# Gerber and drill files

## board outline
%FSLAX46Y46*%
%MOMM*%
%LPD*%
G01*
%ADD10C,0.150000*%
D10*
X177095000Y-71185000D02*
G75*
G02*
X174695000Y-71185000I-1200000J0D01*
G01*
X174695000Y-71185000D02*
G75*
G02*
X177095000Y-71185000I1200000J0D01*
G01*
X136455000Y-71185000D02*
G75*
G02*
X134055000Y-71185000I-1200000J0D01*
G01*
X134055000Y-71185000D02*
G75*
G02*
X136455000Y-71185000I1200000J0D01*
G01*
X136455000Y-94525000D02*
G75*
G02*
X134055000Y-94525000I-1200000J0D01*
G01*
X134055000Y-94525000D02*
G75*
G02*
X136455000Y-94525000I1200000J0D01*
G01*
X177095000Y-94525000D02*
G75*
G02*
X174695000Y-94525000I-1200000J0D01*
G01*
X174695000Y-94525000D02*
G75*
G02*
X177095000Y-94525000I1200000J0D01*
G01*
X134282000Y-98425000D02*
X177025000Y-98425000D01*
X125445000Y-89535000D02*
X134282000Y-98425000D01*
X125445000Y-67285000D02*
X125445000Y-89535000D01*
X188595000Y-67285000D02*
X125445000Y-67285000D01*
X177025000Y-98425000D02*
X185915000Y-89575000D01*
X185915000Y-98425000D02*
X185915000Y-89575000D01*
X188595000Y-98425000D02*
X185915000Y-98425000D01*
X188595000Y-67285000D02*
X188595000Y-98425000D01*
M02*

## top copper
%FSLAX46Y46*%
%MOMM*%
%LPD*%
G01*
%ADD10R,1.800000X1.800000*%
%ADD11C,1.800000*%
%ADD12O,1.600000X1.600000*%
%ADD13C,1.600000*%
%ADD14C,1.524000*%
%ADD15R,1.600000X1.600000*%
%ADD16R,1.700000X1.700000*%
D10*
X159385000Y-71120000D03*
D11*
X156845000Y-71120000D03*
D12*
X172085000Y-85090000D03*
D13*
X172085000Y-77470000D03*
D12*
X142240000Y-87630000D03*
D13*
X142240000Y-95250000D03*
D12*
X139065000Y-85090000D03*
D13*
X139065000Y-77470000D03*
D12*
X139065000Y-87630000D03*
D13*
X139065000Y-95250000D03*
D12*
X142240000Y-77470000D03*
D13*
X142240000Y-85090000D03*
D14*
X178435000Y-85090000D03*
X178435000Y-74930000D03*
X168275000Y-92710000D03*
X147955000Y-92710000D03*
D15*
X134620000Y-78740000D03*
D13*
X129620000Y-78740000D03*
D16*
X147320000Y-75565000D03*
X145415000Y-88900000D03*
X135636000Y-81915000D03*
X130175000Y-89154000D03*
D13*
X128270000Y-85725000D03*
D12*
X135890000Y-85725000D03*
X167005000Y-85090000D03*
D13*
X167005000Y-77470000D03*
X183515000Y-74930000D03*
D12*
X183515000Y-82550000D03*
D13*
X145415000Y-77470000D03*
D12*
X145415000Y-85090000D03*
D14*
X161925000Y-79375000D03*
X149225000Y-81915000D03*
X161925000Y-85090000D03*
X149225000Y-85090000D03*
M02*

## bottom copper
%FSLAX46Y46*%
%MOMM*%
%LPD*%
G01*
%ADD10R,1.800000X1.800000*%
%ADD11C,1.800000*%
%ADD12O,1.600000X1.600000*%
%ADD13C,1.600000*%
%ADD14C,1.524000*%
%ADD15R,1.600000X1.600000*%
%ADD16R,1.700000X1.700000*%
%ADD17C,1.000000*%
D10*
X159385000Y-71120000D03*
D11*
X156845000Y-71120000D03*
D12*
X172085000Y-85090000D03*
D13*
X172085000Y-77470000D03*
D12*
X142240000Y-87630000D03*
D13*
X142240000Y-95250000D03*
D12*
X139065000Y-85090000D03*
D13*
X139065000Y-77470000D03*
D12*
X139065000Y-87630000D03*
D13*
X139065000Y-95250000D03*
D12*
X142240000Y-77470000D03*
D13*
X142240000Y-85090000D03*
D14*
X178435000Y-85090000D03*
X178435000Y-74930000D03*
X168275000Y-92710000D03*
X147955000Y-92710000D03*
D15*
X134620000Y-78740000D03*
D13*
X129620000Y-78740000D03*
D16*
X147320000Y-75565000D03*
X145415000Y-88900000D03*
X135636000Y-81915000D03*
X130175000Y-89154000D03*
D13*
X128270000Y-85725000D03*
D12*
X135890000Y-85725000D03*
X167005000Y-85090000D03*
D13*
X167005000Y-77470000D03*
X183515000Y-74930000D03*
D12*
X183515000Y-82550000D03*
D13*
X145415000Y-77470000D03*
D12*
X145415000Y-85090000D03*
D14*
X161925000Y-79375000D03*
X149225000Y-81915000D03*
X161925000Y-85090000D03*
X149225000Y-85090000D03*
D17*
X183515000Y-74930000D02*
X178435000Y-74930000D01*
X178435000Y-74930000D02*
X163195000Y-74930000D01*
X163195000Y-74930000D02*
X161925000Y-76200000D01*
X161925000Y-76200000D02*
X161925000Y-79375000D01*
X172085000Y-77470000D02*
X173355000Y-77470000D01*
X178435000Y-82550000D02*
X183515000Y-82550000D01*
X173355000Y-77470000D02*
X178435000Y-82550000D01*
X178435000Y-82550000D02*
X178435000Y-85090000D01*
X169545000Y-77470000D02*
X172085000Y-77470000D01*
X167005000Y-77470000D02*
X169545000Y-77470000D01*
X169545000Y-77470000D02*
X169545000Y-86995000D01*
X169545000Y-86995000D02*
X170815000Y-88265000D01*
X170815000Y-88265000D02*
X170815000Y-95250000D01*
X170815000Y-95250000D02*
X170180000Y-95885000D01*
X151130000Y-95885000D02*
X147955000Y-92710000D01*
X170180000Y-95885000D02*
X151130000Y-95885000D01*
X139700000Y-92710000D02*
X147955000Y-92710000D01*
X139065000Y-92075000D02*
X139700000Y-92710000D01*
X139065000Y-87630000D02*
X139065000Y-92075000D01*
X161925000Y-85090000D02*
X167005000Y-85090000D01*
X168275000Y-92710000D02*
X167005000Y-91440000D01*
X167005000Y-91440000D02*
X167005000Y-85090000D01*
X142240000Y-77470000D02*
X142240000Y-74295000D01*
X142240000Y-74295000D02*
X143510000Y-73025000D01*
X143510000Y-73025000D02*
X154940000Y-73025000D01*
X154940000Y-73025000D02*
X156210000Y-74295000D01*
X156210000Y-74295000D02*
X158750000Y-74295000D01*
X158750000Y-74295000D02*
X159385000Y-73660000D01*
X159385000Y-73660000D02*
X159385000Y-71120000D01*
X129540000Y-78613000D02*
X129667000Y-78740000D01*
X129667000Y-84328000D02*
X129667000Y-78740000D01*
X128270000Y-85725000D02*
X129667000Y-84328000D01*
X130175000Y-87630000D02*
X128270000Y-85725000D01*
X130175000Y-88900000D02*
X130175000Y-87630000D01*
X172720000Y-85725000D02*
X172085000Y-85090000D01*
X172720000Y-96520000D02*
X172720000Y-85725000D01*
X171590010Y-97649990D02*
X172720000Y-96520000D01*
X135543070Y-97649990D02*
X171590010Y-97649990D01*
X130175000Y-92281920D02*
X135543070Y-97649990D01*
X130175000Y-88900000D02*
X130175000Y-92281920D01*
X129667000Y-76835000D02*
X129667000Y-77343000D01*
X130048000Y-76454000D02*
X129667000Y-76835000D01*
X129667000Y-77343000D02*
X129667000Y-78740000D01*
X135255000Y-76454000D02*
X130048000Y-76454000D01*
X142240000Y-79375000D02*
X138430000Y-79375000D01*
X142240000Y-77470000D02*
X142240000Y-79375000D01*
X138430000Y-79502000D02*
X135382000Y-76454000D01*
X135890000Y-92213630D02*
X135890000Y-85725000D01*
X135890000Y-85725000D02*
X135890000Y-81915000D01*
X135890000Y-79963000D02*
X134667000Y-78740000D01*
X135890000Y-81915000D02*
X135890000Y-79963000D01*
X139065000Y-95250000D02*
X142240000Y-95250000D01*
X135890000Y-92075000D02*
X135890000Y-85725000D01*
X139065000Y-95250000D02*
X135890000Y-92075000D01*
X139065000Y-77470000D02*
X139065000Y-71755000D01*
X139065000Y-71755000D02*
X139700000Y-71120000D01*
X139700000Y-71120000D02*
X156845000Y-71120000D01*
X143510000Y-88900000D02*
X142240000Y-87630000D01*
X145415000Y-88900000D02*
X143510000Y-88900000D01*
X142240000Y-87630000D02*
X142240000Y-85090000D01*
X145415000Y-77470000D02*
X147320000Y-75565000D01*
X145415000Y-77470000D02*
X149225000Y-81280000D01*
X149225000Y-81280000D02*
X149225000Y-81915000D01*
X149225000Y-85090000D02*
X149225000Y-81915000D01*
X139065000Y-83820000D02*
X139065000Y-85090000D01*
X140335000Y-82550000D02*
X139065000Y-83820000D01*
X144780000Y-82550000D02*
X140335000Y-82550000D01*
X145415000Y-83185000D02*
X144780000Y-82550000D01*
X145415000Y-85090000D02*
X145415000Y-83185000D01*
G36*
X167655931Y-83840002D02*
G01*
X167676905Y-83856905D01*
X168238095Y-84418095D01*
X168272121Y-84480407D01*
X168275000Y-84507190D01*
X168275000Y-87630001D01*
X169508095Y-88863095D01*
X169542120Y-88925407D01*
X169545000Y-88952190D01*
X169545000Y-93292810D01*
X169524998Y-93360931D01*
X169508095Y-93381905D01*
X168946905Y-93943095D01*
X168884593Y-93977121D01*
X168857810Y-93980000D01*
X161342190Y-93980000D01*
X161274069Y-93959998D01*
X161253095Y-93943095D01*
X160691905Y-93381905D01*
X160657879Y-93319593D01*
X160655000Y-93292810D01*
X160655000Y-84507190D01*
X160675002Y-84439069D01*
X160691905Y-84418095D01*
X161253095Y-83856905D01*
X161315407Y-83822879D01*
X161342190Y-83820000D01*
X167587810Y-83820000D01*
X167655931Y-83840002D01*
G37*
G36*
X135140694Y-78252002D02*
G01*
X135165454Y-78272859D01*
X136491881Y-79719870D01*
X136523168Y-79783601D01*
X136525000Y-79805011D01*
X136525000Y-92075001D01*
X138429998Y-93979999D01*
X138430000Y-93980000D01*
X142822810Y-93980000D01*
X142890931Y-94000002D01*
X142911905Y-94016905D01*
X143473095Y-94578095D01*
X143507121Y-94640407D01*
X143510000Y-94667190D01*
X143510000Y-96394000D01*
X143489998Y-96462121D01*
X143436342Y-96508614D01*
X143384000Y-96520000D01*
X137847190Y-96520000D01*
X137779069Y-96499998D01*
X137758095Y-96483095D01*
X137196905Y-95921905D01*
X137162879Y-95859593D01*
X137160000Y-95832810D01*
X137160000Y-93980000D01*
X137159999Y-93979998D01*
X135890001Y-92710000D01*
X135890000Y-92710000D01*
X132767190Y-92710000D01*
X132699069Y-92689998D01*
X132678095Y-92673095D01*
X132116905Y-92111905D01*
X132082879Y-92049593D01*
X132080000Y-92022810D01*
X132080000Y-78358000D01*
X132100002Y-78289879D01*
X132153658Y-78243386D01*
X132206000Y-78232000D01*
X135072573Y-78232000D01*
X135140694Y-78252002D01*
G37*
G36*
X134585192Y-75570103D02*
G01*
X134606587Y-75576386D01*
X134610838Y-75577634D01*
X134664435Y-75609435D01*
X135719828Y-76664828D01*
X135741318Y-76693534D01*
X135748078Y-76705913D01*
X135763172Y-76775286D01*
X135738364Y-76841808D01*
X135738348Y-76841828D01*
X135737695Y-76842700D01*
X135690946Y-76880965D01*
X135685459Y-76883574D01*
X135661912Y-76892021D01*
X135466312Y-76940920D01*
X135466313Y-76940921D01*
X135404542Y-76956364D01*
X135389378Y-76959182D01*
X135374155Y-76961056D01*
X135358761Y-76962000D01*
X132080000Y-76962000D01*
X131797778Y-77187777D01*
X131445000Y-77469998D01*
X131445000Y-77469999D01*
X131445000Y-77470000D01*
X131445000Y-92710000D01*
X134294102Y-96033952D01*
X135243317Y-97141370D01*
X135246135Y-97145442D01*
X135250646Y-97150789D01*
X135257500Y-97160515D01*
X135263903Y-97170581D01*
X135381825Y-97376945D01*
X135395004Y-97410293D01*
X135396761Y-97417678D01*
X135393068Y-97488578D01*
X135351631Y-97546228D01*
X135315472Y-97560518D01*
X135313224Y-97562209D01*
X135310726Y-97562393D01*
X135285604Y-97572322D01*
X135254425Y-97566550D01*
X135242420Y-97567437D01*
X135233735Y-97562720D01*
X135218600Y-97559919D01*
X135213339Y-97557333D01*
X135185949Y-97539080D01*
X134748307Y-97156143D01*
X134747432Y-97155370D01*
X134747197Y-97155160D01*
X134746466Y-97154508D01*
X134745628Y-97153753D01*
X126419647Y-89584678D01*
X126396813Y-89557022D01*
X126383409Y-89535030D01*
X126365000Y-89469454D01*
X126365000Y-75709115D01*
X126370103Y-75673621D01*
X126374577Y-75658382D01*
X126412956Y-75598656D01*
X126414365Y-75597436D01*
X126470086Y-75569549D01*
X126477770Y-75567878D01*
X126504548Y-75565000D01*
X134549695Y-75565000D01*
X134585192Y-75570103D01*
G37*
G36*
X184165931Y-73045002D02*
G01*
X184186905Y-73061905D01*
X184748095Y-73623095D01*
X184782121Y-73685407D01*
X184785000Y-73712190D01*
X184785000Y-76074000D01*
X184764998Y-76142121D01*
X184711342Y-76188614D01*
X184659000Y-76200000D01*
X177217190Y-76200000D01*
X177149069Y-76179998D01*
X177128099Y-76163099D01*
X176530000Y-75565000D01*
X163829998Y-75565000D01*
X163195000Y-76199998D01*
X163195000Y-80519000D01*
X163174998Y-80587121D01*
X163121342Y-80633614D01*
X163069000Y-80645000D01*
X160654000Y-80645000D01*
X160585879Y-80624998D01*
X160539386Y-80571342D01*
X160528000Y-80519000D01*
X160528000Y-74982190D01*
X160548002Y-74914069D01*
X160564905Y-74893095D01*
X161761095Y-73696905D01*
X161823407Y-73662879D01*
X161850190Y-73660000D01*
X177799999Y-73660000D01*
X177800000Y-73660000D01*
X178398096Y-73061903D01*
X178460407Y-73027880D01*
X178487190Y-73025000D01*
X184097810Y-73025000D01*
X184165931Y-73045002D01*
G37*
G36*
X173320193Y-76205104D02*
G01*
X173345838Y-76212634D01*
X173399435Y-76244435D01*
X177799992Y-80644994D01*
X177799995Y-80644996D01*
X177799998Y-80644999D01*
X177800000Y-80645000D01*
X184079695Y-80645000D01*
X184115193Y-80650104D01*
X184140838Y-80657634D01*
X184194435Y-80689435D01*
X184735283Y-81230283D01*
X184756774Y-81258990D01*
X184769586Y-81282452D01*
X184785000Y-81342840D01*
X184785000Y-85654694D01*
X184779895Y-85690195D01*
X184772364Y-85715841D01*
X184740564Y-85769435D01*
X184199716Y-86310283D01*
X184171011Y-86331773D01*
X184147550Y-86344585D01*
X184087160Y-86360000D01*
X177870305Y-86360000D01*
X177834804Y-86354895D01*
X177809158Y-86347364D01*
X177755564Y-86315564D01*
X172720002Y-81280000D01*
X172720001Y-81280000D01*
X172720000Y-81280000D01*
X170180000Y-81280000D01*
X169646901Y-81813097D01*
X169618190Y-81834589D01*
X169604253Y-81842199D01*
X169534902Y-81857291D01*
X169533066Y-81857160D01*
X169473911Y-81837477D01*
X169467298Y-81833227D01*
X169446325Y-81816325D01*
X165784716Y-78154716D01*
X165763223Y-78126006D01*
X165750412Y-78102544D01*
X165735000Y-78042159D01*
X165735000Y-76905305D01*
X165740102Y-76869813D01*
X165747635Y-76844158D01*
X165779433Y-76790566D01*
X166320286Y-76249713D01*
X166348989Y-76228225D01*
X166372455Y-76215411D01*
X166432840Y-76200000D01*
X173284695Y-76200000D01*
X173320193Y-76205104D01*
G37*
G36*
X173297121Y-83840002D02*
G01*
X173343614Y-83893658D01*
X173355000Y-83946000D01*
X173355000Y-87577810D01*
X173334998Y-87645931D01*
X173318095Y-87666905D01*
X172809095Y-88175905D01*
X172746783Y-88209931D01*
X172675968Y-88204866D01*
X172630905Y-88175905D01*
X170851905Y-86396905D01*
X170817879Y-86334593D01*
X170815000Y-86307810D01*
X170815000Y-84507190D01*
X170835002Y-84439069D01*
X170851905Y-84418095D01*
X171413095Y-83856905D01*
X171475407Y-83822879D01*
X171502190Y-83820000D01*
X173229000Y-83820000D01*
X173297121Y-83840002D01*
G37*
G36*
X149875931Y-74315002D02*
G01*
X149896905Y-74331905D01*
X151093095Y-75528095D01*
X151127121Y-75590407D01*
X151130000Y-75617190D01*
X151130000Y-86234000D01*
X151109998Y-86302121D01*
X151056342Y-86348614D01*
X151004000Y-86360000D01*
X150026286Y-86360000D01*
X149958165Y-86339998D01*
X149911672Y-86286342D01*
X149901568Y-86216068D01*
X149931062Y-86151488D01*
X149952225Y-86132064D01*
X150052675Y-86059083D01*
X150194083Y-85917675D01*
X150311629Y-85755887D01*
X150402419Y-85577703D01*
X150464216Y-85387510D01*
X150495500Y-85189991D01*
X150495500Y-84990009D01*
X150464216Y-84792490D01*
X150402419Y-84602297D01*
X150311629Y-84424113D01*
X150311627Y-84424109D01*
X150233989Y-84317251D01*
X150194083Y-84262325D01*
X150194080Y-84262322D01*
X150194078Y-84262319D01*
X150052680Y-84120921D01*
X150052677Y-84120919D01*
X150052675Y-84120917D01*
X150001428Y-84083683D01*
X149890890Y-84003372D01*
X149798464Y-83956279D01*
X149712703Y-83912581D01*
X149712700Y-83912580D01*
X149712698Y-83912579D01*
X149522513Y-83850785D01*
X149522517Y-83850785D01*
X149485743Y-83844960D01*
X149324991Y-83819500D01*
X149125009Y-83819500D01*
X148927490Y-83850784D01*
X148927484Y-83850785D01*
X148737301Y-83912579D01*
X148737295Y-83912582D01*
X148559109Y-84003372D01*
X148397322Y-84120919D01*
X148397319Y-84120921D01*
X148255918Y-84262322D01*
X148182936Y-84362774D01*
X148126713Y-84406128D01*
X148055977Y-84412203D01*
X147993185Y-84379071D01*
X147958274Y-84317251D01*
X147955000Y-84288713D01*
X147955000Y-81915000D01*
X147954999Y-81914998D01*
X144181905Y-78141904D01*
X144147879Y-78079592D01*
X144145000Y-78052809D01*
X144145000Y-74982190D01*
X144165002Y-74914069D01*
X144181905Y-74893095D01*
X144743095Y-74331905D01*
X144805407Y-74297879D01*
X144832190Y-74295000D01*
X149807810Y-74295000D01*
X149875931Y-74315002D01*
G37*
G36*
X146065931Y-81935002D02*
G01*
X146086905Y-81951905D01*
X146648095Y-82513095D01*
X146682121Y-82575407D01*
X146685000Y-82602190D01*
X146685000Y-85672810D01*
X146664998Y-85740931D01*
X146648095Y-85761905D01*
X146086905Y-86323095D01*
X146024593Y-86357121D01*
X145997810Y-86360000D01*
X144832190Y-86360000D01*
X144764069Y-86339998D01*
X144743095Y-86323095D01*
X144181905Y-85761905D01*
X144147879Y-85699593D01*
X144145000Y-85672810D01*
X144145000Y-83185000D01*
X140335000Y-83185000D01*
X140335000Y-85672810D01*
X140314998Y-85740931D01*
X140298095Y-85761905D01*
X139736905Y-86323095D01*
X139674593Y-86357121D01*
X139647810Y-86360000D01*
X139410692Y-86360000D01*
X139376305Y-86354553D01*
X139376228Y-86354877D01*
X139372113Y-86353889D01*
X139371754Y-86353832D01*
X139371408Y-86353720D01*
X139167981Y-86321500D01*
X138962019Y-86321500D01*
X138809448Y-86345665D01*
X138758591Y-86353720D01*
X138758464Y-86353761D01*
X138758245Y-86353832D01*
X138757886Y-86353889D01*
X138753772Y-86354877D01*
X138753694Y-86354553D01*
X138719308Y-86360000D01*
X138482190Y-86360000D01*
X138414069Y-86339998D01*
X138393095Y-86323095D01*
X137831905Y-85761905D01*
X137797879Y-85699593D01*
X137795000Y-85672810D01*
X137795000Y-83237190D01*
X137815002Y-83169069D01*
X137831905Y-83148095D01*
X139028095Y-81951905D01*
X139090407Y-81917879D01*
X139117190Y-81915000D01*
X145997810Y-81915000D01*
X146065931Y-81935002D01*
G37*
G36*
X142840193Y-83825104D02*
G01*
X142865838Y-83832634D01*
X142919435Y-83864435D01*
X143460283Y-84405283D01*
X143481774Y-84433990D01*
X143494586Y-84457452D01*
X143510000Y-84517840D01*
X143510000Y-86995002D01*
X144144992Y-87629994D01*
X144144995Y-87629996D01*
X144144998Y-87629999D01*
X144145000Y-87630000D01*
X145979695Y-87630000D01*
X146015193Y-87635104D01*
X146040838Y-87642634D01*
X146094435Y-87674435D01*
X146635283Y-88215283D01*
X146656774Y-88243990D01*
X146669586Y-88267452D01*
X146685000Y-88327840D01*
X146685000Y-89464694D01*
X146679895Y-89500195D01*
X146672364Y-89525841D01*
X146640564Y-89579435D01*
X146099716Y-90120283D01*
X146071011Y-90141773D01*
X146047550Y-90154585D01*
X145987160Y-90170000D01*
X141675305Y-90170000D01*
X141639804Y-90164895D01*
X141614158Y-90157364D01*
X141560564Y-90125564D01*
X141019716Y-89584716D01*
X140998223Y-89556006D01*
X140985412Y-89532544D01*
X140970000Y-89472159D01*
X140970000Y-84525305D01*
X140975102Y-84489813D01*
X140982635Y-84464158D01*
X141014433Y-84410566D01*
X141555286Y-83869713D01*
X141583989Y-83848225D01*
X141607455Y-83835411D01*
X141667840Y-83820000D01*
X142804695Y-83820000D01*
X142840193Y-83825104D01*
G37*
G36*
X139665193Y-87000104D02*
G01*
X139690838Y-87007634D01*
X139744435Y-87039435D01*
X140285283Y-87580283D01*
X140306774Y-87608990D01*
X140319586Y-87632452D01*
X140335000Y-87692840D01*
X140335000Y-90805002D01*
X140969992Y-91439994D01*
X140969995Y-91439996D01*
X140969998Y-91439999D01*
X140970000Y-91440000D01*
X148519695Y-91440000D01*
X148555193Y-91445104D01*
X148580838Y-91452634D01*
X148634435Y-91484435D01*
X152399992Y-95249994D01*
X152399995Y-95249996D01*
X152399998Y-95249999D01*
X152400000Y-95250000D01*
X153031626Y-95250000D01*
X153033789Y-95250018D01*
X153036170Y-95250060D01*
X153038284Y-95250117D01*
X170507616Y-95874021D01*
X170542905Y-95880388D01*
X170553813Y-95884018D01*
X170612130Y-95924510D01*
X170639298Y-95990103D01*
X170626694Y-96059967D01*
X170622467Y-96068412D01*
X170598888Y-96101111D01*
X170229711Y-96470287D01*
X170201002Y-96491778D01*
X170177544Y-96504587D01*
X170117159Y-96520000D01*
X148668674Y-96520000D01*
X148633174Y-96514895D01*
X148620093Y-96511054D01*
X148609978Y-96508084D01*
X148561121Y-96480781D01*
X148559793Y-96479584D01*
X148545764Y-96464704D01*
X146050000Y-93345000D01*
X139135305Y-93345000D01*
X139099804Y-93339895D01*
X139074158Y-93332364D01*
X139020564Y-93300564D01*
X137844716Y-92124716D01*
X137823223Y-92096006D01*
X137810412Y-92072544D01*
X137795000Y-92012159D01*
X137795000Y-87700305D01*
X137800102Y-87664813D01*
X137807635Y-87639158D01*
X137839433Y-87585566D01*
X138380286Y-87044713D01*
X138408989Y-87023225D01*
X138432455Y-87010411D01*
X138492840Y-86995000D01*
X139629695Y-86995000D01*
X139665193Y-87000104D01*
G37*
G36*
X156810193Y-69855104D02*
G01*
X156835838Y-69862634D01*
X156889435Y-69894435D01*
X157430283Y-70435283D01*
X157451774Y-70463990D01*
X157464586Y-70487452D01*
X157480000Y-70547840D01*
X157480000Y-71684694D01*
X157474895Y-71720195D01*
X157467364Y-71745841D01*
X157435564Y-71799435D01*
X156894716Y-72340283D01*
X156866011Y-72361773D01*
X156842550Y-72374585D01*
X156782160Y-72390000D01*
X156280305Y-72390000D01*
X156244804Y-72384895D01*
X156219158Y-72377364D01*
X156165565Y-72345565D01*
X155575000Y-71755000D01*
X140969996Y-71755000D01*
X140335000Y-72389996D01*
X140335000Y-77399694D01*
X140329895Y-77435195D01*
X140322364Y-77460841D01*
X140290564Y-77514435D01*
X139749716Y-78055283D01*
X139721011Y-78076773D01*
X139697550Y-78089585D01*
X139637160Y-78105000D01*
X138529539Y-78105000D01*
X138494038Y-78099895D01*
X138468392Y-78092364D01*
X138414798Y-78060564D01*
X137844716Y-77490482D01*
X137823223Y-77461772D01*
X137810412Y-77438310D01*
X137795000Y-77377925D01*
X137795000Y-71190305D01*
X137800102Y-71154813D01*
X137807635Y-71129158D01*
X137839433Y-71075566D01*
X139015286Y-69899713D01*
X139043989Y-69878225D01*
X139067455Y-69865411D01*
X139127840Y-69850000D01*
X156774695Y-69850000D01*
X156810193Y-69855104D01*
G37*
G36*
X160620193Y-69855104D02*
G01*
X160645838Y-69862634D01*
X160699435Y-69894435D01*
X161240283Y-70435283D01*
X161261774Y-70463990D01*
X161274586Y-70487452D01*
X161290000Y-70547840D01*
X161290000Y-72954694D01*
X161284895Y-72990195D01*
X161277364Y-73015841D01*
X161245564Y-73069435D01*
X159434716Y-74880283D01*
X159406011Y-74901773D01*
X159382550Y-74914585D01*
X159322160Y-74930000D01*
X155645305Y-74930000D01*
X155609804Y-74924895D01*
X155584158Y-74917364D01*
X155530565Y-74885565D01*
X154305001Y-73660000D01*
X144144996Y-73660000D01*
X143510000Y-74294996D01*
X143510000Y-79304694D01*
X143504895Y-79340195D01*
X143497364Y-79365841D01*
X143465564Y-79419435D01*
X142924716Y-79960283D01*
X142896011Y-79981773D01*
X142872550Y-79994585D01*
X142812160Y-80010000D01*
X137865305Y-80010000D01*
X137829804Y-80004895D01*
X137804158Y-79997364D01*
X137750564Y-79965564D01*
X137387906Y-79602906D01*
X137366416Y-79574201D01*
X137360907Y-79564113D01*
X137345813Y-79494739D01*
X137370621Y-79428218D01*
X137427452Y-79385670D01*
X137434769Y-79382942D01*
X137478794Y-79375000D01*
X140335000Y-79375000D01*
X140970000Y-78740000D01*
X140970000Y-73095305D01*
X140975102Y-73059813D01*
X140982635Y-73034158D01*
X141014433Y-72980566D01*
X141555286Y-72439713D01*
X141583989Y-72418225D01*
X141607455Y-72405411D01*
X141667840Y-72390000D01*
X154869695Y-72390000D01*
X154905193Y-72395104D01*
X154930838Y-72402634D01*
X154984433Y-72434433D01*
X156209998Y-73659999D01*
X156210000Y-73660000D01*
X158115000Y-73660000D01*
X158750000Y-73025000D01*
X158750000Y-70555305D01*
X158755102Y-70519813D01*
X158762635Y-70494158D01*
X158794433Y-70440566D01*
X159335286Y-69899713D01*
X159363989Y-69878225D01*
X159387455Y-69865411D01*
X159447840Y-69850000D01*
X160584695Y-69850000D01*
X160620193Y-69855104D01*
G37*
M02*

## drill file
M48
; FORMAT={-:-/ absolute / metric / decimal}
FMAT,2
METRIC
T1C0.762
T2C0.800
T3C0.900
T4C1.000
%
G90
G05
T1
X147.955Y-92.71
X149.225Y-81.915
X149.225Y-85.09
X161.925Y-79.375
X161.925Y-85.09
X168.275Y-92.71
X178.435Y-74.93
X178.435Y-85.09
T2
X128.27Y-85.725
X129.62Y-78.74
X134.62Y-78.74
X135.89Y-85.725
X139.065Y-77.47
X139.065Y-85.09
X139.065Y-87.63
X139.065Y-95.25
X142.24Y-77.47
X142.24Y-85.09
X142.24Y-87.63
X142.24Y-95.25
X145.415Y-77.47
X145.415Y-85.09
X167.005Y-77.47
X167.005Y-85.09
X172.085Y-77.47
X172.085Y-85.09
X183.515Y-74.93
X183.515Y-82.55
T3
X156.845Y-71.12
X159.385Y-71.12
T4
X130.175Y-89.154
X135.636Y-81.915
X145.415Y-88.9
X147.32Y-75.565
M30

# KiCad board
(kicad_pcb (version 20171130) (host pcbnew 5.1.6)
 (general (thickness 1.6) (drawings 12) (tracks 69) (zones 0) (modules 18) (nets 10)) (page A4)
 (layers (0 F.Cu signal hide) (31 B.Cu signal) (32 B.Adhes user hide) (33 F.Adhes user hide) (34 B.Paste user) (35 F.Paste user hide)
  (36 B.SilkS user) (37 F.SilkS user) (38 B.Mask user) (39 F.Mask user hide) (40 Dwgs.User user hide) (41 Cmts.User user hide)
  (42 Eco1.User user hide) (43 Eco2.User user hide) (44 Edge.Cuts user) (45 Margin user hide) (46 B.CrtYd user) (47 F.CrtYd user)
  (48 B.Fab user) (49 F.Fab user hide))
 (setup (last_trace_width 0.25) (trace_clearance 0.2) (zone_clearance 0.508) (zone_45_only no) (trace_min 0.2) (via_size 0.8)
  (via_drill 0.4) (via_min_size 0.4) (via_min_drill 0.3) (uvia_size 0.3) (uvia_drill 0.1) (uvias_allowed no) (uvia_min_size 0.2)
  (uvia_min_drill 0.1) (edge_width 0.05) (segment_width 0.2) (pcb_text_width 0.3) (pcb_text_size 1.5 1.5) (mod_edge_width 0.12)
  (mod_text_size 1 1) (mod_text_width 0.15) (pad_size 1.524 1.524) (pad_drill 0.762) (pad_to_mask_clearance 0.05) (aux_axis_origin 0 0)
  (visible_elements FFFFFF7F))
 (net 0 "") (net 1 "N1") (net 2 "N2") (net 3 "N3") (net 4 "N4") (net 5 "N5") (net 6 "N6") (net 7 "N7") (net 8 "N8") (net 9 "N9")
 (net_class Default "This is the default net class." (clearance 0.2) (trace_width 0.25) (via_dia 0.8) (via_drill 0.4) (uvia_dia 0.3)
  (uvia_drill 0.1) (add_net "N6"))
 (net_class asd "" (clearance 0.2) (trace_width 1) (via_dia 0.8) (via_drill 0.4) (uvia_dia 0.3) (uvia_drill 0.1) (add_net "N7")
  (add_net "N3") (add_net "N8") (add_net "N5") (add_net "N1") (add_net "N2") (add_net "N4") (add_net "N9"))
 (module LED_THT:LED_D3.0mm (layer F.Cu) (at 159.385 71.12 180)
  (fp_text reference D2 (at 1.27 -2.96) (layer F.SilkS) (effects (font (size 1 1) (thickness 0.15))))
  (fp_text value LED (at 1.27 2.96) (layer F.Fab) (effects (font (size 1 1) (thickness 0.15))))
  (pad 1 thru_hole rect (at 0 0 180) (size 1.8 1.8) (drill 0.9) (layers *.Cu *.Mask) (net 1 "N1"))
  (pad 2 thru_hole circle (at 2.54 0 180) (size 1.8 1.8) (drill 0.9) (layers *.Cu *.Mask) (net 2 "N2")))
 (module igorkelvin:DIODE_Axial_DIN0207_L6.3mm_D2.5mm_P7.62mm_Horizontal (layer F.Cu) (at 172.085 77.47 270)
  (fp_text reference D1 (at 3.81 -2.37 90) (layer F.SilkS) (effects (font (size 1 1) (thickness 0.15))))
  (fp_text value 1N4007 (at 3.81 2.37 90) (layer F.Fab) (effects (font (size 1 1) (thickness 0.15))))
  (pad 2 thru_hole oval (at 7.62 0 270) (size 1.6 1.6) (drill 0.8) (layers *.Cu *.Mask) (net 1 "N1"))
  (pad 1 thru_hole circle (at 0 0 270) (size 1.6 1.6) (drill 0.8) (layers *.Cu *.Mask) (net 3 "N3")))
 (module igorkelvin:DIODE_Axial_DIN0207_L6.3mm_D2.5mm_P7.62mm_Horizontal (layer F.Cu) (at 142.24 95.25 90)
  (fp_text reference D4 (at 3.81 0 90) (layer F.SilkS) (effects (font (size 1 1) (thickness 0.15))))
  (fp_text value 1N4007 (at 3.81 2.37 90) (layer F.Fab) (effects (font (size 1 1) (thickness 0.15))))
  (pad 2 thru_hole oval (at 7.62 0 90) (size 1.6 1.6) (drill 0.8) (layers *.Cu *.Mask) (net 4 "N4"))
  (pad 1 thru_hole circle (at 0 0 90) (size 1.6 1.6) (drill 0.8) (layers *.Cu *.Mask) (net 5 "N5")))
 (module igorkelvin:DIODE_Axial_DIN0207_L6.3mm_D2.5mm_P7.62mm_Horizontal (layer F.Cu) (at 139.065 77.47 270)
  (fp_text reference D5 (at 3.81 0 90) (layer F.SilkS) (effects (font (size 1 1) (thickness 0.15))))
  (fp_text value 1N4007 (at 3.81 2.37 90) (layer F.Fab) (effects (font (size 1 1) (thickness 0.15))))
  (pad 2 thru_hole oval (at 7.62 0 270) (size 1.6 1.6) (drill 0.8) (layers *.Cu *.Mask) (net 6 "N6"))
  (pad 1 thru_hole circle (at 0 0 270) (size 1.6 1.6) (drill 0.8) (layers *.Cu *.Mask) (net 2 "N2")))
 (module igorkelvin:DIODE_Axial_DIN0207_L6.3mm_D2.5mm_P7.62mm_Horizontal (layer F.Cu) (at 139.065 95.25 90)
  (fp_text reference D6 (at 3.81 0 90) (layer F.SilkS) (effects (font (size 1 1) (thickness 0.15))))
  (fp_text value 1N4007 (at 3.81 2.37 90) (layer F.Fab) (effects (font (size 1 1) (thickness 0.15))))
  (pad 2 thru_hole oval (at 7.62 0 90) (size 1.6 1.6) (drill 0.8) (layers *.Cu *.Mask) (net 3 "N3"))
  (pad 1 thru_hole circle (at 0 0 90) (size 1.6 1.6) (drill 0.8) (layers *.Cu *.Mask) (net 5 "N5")))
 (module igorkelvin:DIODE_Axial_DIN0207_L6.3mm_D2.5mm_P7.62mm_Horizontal (layer F.Cu) (at 142.24 85.09 90)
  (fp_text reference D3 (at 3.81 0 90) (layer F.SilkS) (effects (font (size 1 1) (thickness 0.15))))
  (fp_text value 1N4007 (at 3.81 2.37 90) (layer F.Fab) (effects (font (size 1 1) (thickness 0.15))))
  (pad 2 thru_hole oval (at 7.62 0 90) (size 1.6 1.6) (drill 0.8) (layers *.Cu *.Mask) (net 1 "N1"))
  (pad 1 thru_hole circle (at 0 0 90) (size 1.6 1.6) (drill 0.8) (layers *.Cu *.Mask) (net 4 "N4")))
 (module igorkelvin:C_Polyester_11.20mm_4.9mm (layer F.Cu) (at 178.435 74.93 270)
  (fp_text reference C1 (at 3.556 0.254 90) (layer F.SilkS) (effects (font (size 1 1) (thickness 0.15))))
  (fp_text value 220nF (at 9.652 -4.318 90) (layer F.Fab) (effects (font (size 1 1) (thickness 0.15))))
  (pad 2 thru_hole circle (at 10.16 0 270) (size 1.524 1.524) (drill 0.762) (layers *.Cu *.Mask) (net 3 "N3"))
  (pad 1 thru_hole circle (at 0 0 270) (size 1.524 1.524) (drill 0.762) (layers *.Cu *.Mask) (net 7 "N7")))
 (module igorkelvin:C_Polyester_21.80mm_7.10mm (layer F.Cu) (at 168.275 92.71 180)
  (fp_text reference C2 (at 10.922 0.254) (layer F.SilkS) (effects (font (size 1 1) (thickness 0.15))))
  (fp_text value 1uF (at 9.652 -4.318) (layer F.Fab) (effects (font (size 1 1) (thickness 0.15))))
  (pad 1 thru_hole circle (at 0 0 180) (size 1.524 1.524) (drill 0.762) (layers *.Cu *.Mask) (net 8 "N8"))
  (pad 2 thru_hole circle (at 20.32 0 180) (size 1.524 1.524) (drill 0.762) (layers *.Cu *.Mask) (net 3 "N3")))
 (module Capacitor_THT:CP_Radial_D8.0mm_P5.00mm (layer F.Cu) (at 134.62 78.74 180)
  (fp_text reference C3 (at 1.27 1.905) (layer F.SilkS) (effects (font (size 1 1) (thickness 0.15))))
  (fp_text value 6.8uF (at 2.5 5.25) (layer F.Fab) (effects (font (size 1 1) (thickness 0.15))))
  (pad 1 thru_hole rect (at 0 0 180) (size 1.6 1.6) (drill 0.8) (layers *.Cu *.Mask) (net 5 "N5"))
  (pad 2 thru_hole circle (at 5 0 180) (size 1.6 1.6) (drill 0.8) (layers *.Cu *.Mask) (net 1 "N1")))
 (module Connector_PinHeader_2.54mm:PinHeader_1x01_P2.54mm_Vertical (layer F.Cu) (at 147.32 75.565)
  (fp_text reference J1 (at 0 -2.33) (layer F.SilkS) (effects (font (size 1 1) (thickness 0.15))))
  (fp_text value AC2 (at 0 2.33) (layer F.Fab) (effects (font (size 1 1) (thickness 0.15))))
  (pad 1 thru_hole rect (at 0 0) (size 1.7 1.7) (drill 1) (layers *.Cu *.Mask) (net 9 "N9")))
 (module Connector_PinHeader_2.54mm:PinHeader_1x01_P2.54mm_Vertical (layer F.Cu) (at 145.415 88.9)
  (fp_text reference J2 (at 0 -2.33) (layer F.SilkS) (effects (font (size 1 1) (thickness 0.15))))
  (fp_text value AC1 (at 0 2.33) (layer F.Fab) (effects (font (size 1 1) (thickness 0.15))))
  (pad 1 thru_hole rect (at 0 0) (size 1.7 1.7) (drill 1) (layers *.Cu *.Mask) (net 4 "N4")))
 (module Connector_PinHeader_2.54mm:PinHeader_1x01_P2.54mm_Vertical (layer F.Cu) (at 135.636 81.915)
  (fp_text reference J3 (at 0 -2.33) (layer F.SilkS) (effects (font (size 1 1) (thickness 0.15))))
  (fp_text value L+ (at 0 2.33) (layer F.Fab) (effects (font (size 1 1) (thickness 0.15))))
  (pad 1 thru_hole rect (at 0 0) (size 1.7 1.7) (drill 1) (layers *.Cu *.Mask) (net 5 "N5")))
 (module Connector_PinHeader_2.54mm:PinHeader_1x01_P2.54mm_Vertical (layer F.Cu) (at 130.175 89.154)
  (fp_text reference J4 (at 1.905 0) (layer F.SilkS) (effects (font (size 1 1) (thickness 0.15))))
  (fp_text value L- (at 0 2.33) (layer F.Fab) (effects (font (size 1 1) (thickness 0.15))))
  (pad 1 thru_hole rect (at 0 0) (size 1.7 1.7) (drill 1) (layers *.Cu *.Mask) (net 1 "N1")))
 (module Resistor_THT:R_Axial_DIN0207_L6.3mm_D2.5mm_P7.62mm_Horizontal (layer F.Cu) (at 128.27 85.725)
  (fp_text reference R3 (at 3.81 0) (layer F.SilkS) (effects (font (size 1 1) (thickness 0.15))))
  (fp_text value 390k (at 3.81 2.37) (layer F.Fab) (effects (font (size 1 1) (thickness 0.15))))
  (pad 1 thru_hole circle (at 0 0) (size 1.6 1.6) (drill 0.8) (layers *.Cu *.Mask) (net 1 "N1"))
  (pad 2 thru_hole oval (at 7.62 0) (size 1.6 1.6) (drill 0.8) (layers *.Cu *.Mask) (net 5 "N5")))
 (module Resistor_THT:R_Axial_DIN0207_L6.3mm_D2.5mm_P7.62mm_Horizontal (layer F.Cu) (at 167.005 77.47 270)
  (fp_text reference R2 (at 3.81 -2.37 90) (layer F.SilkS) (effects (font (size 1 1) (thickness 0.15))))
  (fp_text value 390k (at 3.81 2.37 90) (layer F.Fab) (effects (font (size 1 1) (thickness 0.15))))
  (pad 2 thru_hole oval (at 7.62 0 270) (size 1.6 1.6) (drill 0.8) (layers *.Cu *.Mask) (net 8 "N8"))
  (pad 1 thru_hole circle (at 0 0 270) (size 1.6 1.6) (drill 0.8) (layers *.Cu *.Mask) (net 3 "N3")))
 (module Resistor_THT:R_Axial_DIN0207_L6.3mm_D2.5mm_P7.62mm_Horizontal (layer F.Cu) (at 183.515 74.93 270)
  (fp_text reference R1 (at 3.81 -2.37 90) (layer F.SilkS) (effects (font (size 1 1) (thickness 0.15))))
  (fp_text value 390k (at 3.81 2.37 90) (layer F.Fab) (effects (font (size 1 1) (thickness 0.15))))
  (pad 1 thru_hole circle (at 0 0 270) (size 1.6 1.6) (drill 0.8) (layers *.Cu *.Mask) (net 7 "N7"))
  (pad 2 thru_hole oval (at 7.62 0 270) (size 1.6 1.6) (drill 0.8) (layers *.Cu *.Mask) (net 3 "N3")))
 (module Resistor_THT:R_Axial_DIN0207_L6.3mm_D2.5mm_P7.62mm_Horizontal (layer F.Cu) (at 145.415 77.47 270)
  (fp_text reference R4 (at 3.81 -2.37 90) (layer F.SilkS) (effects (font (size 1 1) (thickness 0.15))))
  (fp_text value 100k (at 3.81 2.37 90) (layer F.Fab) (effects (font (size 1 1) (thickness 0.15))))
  (pad 1 thru_hole circle (at 0 0 270) (size 1.6 1.6) (drill 0.8) (layers *.Cu *.Mask) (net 9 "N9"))
  (pad 2 thru_hole oval (at 7.62 0 270) (size 1.6 1.6) (drill 0.8) (layers *.Cu *.Mask) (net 6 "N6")))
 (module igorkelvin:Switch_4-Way (layer F.Cu) (at 149.225 85.09)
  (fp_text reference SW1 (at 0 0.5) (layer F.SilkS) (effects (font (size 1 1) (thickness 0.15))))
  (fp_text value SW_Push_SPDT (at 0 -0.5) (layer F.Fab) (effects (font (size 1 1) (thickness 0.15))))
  (pad 1 thru_hole circle (at 12.7 -5.715) (size 1.524 1.524) (drill 0.762) (layers *.Cu *.Mask) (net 7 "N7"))
  (pad 2 thru_hole circle (at 0 -3.175) (size 1.524 1.524) (drill 0.762) (layers *.Cu *.Mask) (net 9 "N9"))
  (pad 3 thru_hole circle (at 12.7 0) (size 1.524 1.524) (drill 0.762) (layers *.Cu *.Mask) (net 8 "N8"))
  (pad 4 thru_hole circle (at 0 0) (size 1.524 1.524) (drill 0.762) (layers *.Cu *.Mask)))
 (gr_circle (center 175.895 71.185) (end 177.095 71.185) (layer Edge.Cuts) (width 0.15))
 (gr_circle (center 135.255 71.185) (end 136.455 71.185) (layer Edge.Cuts) (width 0.15))
 (gr_circle (center 135.255 94.525) (end 136.455 94.525) (layer Edge.Cuts) (width 0.15))
 (gr_circle (center 175.895 94.525) (end 177.095 94.525) (layer Edge.Cuts) (width 0.15))
 (gr_line (start 134.282 98.425) (end 177.025 98.425) (layer Edge.Cuts) (width 0.15))
 (gr_line (start 125.445 89.535) (end 134.282 98.425) (layer Edge.Cuts) (width 0.15))
 (gr_line (start 125.445 67.285) (end 125.445 89.535) (layer Edge.Cuts) (width 0.15))
 (gr_line (start 188.595 67.285) (end 125.445 67.285) (layer Edge.Cuts) (width 0.15))
 (gr_line (start 177.025 98.425) (end 185.915 89.575) (layer Edge.Cuts) (width 0.15))
 (gr_line (start 185.915 98.425) (end 185.915 89.575) (layer Edge.Cuts) (width 0.15))
 (gr_line (start 188.595 98.425) (end 185.915 98.425) (layer Edge.Cuts) (width 0.15))
 (gr_line (start 188.595 67.285) (end 188.595 98.425) (layer Edge.Cuts) (width 0.15))
 (segment (start 183.515 74.93) (end 178.435 74.93) (width 1) (layer B.Cu) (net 7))
 (segment (start 178.435 74.93) (end 163.195 74.93) (width 1) (layer B.Cu) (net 7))
 (segment (start 163.195 74.93) (end 161.925 76.2) (width 1) (layer B.Cu) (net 7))
 (segment (start 161.925 76.2) (end 161.925 79.375) (width 1) (layer B.Cu) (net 7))
 (segment (start 172.085 77.47) (end 173.355 77.47) (width 1) (layer B.Cu) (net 3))
 (segment (start 178.435 82.55) (end 183.515 82.55) (width 1) (layer B.Cu) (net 3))
 (segment (start 173.355 77.47) (end 178.435 82.55) (width 1) (layer B.Cu) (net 3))
 (segment (start 178.435 82.55) (end 178.435 85.09) (width 1) (layer B.Cu) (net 3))
 (segment (start 169.545 77.47) (end 172.085 77.47) (width 1) (layer B.Cu) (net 3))
 (segment (start 167.005 77.47) (end 169.545 77.47) (width 1) (layer B.Cu) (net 3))
 (segment (start 169.545 77.47) (end 169.545 86.995) (width 1) (layer B.Cu) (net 3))
 (segment (start 169.545 86.995) (end 170.815 88.265) (width 1) (layer B.Cu) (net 3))
 (segment (start 170.815 88.265) (end 170.815 95.25) (width 1) (layer B.Cu) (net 3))
 (segment (start 170.815 95.25) (end 170.18 95.885) (width 1) (layer B.Cu) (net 3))
 (segment (start 151.13 95.885) (end 147.955 92.71) (width 1) (layer B.Cu) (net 3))
 (segment (start 170.18 95.885) (end 151.13 95.885) (width 1) (layer B.Cu) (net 3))
 (segment (start 139.7 92.71) (end 147.955 92.71) (width 1) (layer B.Cu) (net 3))
 (segment (start 139.065 92.075) (end 139.7 92.71) (width 1) (layer B.Cu) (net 3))
 (segment (start 139.065 87.63) (end 139.065 92.075) (width 1) (layer B.Cu) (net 3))
 (segment (start 161.925 85.09) (end 167.005 85.09) (width 1) (layer B.Cu) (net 8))
 (segment (start 168.275 92.71) (end 167.005 91.44) (width 1) (layer B.Cu) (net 8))
 (segment (start 167.005 91.44) (end 167.005 85.09) (width 1) (layer B.Cu) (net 8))
 (segment (start 142.24 77.47) (end 142.24 74.295) (width 1) (layer B.Cu) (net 1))
 (segment (start 142.24 74.295) (end 143.51 73.025) (width 1) (layer B.Cu) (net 1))
 (segment (start 143.51 73.025) (end 154.94 73.025) (width 1) (layer B.Cu) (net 1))
 (segment (start 154.94 73.025) (end 156.21 74.295) (width 1) (layer B.Cu) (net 1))
 (segment (start 156.21 74.295) (end 158.75 74.295) (width 1) (layer B.Cu) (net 1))
 (segment (start 158.75 74.295) (end 159.385 73.66) (width 1) (layer B.Cu) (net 1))
 (segment (start 159.385 73.66) (end 159.385 71.12) (width 1) (layer B.Cu) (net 1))
 (segment (start 129.54 78.613) (end 129.667 78.74) (width 1) (layer B.Cu) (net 1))
 (segment (start 129.667 84.328) (end 129.667 78.74) (width 1) (layer B.Cu) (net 1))
 (segment (start 128.27 85.725) (end 129.667 84.328) (width 1) (layer B.Cu) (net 1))
 (segment (start 130.175 87.63) (end 128.27 85.725) (width 1) (layer B.Cu) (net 1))
 (segment (start 130.175 88.9) (end 130.175 87.63) (width 1) (layer B.Cu) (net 1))
 (segment (start 172.72 85.725) (end 172.085 85.09) (width 1) (layer B.Cu) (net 1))
 (segment (start 172.72 96.52) (end 172.72 85.725) (width 1) (layer B.Cu) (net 1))
 (segment (start 171.59001 97.64999) (end 172.72 96.52) (width 1) (layer B.Cu) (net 1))
 (segment (start 135.54307 97.64999) (end 171.59001 97.64999) (width 1) (layer B.Cu) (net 1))
 (segment (start 130.175 92.28192) (end 135.54307 97.64999) (width 1) (layer B.Cu) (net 1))
 (segment (start 130.175 88.9) (end 130.175 92.28192) (width 1) (layer B.Cu) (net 1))
 (segment (start 129.667 76.835) (end 129.667 77.343) (width 1) (layer B.Cu) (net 1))
 (segment (start 130.048 76.454) (end 129.667 76.835) (width 1) (layer B.Cu) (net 1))
 (segment (start 129.667 77.343) (end 129.667 78.74) (width 1) (layer B.Cu) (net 1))
 (segment (start 135.255 76.454) (end 130.048 76.454) (width 1) (layer B.Cu) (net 1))
 (segment (start 142.24 79.375) (end 138.43 79.375) (width 1) (layer B.Cu) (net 1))
 (segment (start 142.24 77.47) (end 142.24 79.375) (width 1) (layer B.Cu) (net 1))
 (segment (start 138.43 79.502) (end 135.382 76.454) (width 1) (layer B.Cu) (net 1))
 (segment (start 135.89 92.21363) (end 135.89 85.725) (width 1) (layer B.Cu) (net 5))
 (segment (start 135.89 85.725) (end 135.89 81.915) (width 1) (layer B.Cu) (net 5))
 (segment (start 135.89 79.963) (end 134.667 78.74) (width 1) (layer B.Cu) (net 5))
 (segment (start 135.89 81.915) (end 135.89 79.963) (width 1) (layer B.Cu) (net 5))
 (segment (start 139.065 95.25) (end 142.24 95.25) (width 1) (layer B.Cu) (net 5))
 (segment (start 135.89 92.075) (end 135.89 85.725) (width 1) (layer B.Cu) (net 5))
 (segment (start 139.065 95.25) (end 135.89 92.075) (width 1) (layer B.Cu) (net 5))
 (segment (start 139.065 77.47) (end 139.065 71.755) (width 1) (layer B.Cu) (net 2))
 (segment (start 139.065 71.755) (end 139.7 71.12) (width 1) (layer B.Cu) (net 2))
 (segment (start 139.7 71.12) (end 156.845 71.12) (width 1) (layer B.Cu) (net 2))
 (segment (start 143.51 88.9) (end 142.24 87.63) (width 1) (layer B.Cu) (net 4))
 (segment (start 145.415 88.9) (end 143.51 88.9) (width 1) (layer B.Cu) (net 4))
 (segment (start 142.24 87.63) (end 142.24 85.09) (width 1) (layer B.Cu) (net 4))
 (segment (start 145.415 77.47) (end 147.32 75.565) (width 1) (layer B.Cu) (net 9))
 (segment (start 145.415 77.47) (end 149.225 81.28) (width 1) (layer B.Cu) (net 9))
 (segment (start 149.225 81.28) (end 149.225 81.915) (width 1) (layer B.Cu) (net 9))
 (segment (start 149.225 85.09) (end 149.225 81.915) (width 1) (layer B.Cu) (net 9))
 (segment (start 139.065 83.82) (end 139.065 85.09) (width 1) (layer B.Cu) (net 6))
 (segment (start 140.335 82.55) (end 139.065 83.82) (width 1) (layer B.Cu) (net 6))
 (segment (start 144.78 82.55) (end 140.335 82.55) (width 1) (layer B.Cu) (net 6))
 (segment (start 145.415 83.185) (end 144.78 82.55) (width 1) (layer B.Cu) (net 6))
 (segment (start 145.415 85.09) (end 145.415 83.185) (width 1) (layer B.Cu) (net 6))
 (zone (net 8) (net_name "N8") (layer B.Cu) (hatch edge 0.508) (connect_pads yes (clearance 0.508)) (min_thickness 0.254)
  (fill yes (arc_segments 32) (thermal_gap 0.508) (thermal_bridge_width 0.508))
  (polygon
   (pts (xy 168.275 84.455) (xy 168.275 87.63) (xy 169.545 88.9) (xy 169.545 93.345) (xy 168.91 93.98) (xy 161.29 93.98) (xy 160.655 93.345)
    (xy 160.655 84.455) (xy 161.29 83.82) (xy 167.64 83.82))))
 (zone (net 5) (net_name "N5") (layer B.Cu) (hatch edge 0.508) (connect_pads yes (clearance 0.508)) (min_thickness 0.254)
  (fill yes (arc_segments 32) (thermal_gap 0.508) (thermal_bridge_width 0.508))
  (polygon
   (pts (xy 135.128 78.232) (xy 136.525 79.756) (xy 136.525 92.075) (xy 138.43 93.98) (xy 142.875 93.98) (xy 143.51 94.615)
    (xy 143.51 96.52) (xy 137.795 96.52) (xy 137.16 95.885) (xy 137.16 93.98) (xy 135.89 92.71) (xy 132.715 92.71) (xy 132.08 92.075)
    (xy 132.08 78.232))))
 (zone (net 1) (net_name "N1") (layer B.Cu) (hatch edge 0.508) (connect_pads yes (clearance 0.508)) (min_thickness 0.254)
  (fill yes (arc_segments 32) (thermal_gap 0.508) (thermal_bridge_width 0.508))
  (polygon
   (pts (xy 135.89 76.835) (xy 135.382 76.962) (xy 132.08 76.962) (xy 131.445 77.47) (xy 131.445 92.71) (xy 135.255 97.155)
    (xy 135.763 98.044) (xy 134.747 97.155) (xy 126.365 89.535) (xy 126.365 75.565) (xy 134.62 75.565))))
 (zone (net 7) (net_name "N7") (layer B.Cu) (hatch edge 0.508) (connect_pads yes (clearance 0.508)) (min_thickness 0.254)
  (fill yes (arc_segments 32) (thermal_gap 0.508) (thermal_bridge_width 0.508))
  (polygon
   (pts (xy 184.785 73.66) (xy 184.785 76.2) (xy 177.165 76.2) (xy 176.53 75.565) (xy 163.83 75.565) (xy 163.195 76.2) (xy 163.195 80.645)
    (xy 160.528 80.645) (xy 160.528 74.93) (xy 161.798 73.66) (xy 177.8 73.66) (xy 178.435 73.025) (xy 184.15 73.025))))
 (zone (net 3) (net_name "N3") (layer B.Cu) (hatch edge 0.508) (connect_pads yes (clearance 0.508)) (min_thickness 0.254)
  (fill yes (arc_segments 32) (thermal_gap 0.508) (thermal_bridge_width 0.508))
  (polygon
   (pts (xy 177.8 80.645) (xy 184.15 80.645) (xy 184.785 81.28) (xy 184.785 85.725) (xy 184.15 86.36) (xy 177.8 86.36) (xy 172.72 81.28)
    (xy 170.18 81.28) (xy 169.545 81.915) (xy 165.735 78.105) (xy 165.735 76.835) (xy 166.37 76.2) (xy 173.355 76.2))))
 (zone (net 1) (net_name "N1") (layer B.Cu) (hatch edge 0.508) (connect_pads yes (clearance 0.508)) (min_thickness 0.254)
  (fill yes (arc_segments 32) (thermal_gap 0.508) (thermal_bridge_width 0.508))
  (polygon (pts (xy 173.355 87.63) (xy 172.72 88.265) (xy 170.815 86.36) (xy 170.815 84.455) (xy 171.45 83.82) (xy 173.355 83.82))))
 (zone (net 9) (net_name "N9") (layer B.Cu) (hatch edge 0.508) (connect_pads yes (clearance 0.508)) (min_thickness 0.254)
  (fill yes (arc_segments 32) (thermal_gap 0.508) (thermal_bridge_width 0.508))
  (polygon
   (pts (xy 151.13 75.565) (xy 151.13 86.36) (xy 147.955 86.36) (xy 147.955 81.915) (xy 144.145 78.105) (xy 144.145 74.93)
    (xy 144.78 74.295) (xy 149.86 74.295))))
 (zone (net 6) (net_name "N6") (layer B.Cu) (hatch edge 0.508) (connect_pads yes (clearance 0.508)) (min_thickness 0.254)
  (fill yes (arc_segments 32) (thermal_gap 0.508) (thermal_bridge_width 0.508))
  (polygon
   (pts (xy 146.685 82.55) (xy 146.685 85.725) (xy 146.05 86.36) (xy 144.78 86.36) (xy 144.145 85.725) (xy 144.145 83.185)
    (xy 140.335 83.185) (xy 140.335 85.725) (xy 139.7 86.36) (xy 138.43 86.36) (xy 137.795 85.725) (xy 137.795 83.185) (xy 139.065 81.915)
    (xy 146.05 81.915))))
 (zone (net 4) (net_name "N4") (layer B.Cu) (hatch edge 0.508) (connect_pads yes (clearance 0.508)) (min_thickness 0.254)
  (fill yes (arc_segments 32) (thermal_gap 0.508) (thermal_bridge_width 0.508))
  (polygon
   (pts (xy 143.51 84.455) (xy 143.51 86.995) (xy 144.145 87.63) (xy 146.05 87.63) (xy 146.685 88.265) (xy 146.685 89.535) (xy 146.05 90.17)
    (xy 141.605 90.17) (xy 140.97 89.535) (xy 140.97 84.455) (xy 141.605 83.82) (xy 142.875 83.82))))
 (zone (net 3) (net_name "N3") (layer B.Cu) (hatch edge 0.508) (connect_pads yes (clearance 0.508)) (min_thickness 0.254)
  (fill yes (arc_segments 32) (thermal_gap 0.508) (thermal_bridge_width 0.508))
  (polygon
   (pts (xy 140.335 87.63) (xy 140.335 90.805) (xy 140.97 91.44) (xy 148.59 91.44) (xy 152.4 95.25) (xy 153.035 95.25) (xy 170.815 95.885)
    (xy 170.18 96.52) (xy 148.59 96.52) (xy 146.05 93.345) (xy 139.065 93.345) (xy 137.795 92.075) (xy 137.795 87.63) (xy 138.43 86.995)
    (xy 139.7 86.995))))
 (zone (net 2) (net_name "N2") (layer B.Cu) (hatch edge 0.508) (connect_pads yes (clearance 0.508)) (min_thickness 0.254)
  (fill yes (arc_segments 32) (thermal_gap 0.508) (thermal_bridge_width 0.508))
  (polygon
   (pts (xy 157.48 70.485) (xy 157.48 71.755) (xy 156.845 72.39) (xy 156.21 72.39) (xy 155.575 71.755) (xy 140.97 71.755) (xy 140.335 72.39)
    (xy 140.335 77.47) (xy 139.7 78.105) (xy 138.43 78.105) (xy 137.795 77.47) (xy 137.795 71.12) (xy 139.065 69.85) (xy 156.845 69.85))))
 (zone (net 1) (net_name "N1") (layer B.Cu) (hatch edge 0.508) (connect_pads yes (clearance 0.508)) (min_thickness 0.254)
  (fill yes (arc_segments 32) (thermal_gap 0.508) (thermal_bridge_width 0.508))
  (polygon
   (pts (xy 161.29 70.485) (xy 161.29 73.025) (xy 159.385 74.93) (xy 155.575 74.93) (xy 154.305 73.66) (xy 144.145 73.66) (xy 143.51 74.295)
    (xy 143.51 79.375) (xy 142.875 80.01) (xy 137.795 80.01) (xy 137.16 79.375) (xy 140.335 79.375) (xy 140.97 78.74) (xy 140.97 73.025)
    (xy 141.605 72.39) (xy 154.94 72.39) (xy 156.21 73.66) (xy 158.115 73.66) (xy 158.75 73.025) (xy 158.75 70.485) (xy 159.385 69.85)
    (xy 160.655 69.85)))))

